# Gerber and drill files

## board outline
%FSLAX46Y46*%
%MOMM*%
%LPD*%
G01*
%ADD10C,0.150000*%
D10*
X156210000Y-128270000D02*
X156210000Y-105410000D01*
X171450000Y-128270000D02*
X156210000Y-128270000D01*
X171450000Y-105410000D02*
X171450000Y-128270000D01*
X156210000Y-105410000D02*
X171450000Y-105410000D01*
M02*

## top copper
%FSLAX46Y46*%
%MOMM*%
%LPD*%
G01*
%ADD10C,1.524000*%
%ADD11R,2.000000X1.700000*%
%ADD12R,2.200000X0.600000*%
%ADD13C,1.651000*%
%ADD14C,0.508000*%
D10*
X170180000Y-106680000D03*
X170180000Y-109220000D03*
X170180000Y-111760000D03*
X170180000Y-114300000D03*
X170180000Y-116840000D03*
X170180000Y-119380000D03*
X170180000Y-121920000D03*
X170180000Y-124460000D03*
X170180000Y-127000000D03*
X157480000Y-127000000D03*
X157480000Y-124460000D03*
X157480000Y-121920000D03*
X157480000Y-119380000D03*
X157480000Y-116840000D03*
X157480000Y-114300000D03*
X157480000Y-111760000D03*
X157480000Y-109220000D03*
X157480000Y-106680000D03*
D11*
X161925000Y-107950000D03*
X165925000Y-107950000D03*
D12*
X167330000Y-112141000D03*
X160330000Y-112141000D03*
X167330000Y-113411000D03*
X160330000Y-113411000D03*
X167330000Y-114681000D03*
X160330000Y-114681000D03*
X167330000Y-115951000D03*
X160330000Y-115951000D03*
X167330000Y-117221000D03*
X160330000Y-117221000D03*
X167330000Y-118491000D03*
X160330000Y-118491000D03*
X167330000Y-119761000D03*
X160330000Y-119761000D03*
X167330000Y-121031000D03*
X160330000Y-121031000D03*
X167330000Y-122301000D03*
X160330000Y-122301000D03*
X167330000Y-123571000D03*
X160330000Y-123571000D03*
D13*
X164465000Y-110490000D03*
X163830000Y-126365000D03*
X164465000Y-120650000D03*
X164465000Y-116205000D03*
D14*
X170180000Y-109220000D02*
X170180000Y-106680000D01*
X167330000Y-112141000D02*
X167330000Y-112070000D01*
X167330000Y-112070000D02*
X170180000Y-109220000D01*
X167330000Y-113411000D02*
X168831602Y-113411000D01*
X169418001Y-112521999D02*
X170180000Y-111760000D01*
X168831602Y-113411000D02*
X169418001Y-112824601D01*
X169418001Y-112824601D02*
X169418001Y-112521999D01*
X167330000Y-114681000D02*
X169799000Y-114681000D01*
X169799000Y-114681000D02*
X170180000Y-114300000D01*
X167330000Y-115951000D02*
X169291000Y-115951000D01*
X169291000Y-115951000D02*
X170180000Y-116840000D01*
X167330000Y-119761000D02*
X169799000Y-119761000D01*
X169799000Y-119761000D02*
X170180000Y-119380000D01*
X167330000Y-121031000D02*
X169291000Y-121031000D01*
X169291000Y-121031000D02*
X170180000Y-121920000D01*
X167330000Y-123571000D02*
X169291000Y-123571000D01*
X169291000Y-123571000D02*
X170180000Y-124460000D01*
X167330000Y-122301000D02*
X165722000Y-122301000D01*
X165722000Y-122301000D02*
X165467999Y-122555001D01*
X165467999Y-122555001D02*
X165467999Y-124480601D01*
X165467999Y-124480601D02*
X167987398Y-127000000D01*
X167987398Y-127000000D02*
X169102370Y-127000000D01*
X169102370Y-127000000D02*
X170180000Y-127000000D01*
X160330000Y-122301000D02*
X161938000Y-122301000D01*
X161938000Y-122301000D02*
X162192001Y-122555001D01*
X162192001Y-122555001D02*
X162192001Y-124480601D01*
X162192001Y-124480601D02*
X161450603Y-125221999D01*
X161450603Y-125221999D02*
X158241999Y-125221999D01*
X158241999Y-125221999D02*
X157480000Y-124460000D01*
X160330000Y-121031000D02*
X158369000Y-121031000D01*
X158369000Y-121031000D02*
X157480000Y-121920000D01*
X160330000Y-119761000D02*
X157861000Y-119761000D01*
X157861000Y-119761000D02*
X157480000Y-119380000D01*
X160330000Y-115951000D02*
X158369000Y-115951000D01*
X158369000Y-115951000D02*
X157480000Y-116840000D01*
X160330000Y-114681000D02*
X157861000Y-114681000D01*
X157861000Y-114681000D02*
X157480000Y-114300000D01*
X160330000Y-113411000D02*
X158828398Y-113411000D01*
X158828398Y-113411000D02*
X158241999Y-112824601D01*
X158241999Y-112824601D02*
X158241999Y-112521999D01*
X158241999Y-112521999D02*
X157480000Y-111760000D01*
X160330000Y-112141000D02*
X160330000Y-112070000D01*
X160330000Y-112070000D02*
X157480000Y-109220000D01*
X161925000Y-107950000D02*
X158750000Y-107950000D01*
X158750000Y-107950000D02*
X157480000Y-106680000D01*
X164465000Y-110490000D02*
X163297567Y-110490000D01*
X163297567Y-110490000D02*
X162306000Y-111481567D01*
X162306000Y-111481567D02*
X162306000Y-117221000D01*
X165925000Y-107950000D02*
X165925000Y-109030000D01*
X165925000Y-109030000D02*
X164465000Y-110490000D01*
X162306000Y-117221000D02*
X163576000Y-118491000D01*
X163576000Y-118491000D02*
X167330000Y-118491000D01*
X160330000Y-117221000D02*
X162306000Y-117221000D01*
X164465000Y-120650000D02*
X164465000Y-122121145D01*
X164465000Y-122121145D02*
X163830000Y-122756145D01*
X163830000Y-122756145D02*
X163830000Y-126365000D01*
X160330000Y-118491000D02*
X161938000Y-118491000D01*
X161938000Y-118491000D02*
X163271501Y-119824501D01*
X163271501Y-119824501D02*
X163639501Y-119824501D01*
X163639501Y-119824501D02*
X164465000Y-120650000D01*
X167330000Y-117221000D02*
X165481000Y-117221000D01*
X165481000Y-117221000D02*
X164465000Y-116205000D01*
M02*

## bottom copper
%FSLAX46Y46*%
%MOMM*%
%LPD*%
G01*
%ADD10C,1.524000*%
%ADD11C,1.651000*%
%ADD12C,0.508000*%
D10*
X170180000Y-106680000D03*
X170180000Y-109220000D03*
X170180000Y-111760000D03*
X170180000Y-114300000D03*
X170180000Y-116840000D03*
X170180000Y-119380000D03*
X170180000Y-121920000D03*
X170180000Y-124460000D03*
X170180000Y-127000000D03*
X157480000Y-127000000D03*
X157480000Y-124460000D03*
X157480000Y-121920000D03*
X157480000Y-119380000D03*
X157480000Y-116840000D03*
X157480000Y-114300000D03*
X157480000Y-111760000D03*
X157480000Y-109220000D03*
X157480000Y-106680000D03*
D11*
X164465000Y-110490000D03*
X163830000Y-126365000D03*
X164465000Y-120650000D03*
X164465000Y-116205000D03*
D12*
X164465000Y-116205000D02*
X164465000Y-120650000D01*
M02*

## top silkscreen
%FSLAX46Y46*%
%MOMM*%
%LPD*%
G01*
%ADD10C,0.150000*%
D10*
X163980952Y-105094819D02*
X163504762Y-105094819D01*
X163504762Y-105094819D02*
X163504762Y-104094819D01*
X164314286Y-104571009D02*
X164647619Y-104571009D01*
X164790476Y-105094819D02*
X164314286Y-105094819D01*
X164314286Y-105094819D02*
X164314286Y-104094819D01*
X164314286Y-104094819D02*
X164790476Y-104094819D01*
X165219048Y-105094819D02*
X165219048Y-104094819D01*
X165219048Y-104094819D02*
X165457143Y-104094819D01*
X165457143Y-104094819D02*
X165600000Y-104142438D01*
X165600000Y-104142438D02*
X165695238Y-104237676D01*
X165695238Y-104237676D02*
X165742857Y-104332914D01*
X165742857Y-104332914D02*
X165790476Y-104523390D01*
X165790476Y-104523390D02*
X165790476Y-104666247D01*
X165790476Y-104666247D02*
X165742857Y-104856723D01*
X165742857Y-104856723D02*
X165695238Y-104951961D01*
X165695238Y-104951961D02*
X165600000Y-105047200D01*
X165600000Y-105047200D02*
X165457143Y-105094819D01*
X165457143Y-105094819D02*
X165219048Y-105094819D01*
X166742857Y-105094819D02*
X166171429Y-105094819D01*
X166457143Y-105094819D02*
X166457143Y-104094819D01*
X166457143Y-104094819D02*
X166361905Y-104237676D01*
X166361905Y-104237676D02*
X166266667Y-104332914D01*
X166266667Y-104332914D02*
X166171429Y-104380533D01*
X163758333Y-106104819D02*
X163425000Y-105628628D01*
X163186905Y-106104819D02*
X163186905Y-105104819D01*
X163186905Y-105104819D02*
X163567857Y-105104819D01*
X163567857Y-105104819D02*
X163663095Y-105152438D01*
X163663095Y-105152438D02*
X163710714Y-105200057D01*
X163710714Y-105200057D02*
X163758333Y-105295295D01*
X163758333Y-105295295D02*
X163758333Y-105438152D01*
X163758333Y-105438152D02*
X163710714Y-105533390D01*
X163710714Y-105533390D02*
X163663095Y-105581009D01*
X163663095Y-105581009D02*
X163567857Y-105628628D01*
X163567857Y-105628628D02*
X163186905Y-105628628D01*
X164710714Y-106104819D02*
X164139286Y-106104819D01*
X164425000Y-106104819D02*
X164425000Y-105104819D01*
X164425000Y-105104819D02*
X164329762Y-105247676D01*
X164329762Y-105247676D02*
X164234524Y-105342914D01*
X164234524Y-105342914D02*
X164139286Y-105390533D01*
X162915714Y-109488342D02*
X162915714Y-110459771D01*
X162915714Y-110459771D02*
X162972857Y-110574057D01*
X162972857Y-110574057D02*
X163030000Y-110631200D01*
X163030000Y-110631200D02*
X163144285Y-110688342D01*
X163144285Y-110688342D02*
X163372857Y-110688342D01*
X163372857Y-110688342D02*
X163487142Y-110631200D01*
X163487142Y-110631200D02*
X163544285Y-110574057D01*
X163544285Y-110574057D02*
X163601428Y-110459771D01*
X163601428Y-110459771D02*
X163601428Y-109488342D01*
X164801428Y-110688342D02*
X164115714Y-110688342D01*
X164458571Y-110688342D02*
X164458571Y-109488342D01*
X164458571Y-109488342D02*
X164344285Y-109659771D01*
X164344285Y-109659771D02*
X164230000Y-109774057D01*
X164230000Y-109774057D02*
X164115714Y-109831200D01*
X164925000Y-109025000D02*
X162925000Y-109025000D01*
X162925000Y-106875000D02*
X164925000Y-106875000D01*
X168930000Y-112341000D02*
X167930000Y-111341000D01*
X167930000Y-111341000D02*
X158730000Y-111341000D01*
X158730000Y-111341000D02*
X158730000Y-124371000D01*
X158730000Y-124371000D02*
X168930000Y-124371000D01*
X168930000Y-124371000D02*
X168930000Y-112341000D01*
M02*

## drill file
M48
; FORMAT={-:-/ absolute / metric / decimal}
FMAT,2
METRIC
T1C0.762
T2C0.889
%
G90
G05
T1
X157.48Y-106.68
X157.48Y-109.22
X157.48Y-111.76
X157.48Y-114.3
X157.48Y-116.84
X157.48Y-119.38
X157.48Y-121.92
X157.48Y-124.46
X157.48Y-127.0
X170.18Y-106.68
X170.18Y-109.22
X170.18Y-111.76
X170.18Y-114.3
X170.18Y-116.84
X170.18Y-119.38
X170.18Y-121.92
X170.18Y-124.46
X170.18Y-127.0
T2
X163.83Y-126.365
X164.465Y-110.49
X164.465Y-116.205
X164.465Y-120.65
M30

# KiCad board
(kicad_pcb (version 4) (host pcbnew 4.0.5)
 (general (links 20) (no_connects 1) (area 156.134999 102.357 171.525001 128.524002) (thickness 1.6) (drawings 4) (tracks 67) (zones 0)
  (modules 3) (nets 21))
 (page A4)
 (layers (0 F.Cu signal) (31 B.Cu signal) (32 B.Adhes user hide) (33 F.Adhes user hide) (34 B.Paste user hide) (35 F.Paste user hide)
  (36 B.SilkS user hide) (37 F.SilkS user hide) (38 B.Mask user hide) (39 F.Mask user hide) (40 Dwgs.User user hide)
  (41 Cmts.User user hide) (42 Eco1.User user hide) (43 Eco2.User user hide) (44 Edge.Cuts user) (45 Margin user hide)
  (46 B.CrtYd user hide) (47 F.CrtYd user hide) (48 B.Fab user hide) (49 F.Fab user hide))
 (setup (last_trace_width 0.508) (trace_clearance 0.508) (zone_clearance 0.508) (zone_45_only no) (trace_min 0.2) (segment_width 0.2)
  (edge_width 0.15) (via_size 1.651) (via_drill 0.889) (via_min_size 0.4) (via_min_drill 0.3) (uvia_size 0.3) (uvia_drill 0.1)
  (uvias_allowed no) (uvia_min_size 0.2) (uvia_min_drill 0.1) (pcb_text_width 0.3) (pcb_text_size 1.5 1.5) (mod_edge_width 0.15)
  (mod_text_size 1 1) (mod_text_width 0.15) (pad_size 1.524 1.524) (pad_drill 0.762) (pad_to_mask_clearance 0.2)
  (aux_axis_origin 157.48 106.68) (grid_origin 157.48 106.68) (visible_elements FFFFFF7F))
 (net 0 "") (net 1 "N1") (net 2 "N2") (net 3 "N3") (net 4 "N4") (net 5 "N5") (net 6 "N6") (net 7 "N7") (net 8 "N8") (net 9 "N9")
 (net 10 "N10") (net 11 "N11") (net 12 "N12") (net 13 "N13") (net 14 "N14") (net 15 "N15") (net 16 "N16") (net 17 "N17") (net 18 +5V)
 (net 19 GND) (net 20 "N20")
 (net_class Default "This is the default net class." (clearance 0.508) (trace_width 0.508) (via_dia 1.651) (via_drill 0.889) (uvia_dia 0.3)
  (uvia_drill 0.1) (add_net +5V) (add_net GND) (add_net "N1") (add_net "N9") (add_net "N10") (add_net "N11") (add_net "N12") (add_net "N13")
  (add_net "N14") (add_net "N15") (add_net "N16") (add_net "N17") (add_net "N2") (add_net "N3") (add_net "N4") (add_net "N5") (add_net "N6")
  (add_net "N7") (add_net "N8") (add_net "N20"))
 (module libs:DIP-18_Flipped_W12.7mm (layer F.Cu) (at 165.1 104.14)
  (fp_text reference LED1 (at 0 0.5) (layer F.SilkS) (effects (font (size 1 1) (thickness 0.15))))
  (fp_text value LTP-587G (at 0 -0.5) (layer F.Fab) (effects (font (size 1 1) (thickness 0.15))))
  (pad 1 thru_hole circle (at 5.08 2.54) (size 1.524 1.524) (drill 0.762) (layers *.Cu *.Mask) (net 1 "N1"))
  (pad 2 thru_hole circle (at 5.08 5.08) (size 1.524 1.524) (drill 0.762) (layers *.Cu *.Mask) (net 1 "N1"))
  (pad 3 thru_hole circle (at 5.08 7.62) (size 1.524 1.524) (drill 0.762) (layers *.Cu *.Mask) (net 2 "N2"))
  (pad 4 thru_hole circle (at 5.08 10.16) (size 1.524 1.524) (drill 0.762) (layers *.Cu *.Mask) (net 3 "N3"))
  (pad 5 thru_hole circle (at 5.08 12.7) (size 1.524 1.524) (drill 0.762) (layers *.Cu *.Mask) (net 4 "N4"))
  (pad 6 thru_hole circle (at 5.08 15.24) (size 1.524 1.524) (drill 0.762) (layers *.Cu *.Mask) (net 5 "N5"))
  (pad 7 thru_hole circle (at 5.08 17.78) (size 1.524 1.524) (drill 0.762) (layers *.Cu *.Mask) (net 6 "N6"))
  (pad 8 thru_hole circle (at 5.08 20.32) (size 1.524 1.524) (drill 0.762) (layers *.Cu *.Mask) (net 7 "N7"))
  (pad 9 thru_hole circle (at 5.08 22.86) (size 1.524 1.524) (drill 0.762) (layers *.Cu *.Mask) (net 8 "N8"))
  (pad 10 thru_hole circle (at -7.62 22.86) (size 1.524 1.524) (drill 0.762) (layers *.Cu *.Mask) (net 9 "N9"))
  (pad 11 thru_hole circle (at -7.62 20.32) (size 1.524 1.524) (drill 0.762) (layers *.Cu *.Mask) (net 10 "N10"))
  (pad 12 thru_hole circle (at -7.62 17.78) (size 1.524 1.524) (drill 0.762) (layers *.Cu *.Mask) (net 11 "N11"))
  (pad 13 thru_hole circle (at -7.62 15.24) (size 1.524 1.524) (drill 0.762) (layers *.Cu *.Mask) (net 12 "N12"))
  (pad 14 thru_hole circle (at -7.62 12.7) (size 1.524 1.524) (drill 0.762) (layers *.Cu *.Mask) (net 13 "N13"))
  (pad 15 thru_hole circle (at -7.62 10.16) (size 1.524 1.524) (drill 0.762) (layers *.Cu *.Mask) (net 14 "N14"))
  (pad 16 thru_hole circle (at -7.62 7.62) (size 1.524 1.524) (drill 0.762) (layers *.Cu *.Mask) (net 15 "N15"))
  (pad 17 thru_hole circle (at -7.62 5.08) (size 1.524 1.524) (drill 0.762) (layers *.Cu *.Mask) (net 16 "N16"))
  (pad 18 thru_hole circle (at -7.62 2.54) (size 1.524 1.524) (drill 0.762) (layers *.Cu *.Mask) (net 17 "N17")))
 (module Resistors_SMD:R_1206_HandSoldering (layer F.Cu) (at 163.925 107.95)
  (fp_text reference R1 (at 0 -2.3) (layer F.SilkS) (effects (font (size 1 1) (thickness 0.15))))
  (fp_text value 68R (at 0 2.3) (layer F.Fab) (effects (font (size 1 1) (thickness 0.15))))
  (fp_line (start 1 1.075) (end -1 1.075) (layer F.SilkS) (width 0.15))
  (fp_line (start -1 -1.075) (end 1 -1.075) (layer F.SilkS) (width 0.15))
  (pad 1 smd rect (at -2 0) (size 2 1.7) (layers F.Cu F.Paste F.Mask) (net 17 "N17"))
  (pad 2 smd rect (at 2 0) (size 2 1.7) (layers F.Cu F.Paste F.Mask) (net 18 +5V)))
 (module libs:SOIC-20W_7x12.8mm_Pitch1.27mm (layer F.Cu) (at 163.83 117.856 270)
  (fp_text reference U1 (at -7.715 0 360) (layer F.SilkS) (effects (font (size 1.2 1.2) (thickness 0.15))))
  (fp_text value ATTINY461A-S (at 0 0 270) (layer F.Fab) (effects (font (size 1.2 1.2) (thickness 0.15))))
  (fp_line (start -5.515 -5.1) (end -6.515 -4.1) (layer F.SilkS) (width 0.15))
  (fp_line (start -6.515 -4.1) (end -6.515 5.1) (layer F.SilkS) (width 0.15))
  (fp_line (start -6.515 5.1) (end 6.515 5.1) (layer F.SilkS) (width 0.15))
  (fp_line (start 6.515 5.1) (end 6.515 -5.1) (layer F.SilkS) (width 0.15))
  (fp_line (start 6.515 -5.1) (end -5.515 -5.1) (layer F.SilkS) (width 0.15))
  (pad 20 smd rect (at -5.715 -3.5 270) (size 0.6 2.2) (layers F.Cu F.Paste F.Mask) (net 1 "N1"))
  (pad 1 smd rect (at -5.715 3.5 270) (size 0.6 2.2) (layers F.Cu F.Paste F.Mask) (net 16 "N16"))
  (pad 19 smd rect (at -4.445 -3.5 270) (size 0.6 2.2) (layers F.Cu F.Paste F.Mask) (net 2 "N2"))
  (pad 2 smd rect (at -4.445 3.5 270) (size 0.6 2.2) (layers F.Cu F.Paste F.Mask) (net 15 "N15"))
  (pad 18 smd rect (at -3.175 -3.5 270) (size 0.6 2.2) (layers F.Cu F.Paste F.Mask) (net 3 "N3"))
  (pad 3 smd rect (at -3.175 3.5 270) (size 0.6 2.2) (layers F.Cu F.Paste F.Mask) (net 14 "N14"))
  (pad 17 smd rect (at -1.905 -3.5 270) (size 0.6 2.2) (layers F.Cu F.Paste F.Mask) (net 4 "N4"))
  (pad 4 smd rect (at -1.905 3.5 270) (size 0.6 2.2) (layers F.Cu F.Paste F.Mask) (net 13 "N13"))
  (pad 16 smd rect (at -0.635 -3.5 270) (size 0.6 2.2) (layers F.Cu F.Paste F.Mask) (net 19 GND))
  (pad 5 smd rect (at -0.635 3.5 270) (size 0.6 2.2) (layers F.Cu F.Paste F.Mask) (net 18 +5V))
  (pad 15 smd rect (at 0.635 -3.5 270) (size 0.6 2.2) (layers F.Cu F.Paste F.Mask) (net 18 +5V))
  (pad 6 smd rect (at 0.635 3.5 270) (size 0.6 2.2) (layers F.Cu F.Paste F.Mask) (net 19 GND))
  (pad 14 smd rect (at 1.905 -3.5 270) (size 0.6 2.2) (layers F.Cu F.Paste F.Mask) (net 5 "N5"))
  (pad 7 smd rect (at 1.905 3.5 270) (size 0.6 2.2) (layers F.Cu F.Paste F.Mask) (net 12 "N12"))
  (pad 13 smd rect (at 3.175 -3.5 270) (size 0.6 2.2) (layers F.Cu F.Paste F.Mask) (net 6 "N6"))
  (pad 8 smd rect (at 3.175 3.5 270) (size 0.6 2.2) (layers F.Cu F.Paste F.Mask) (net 11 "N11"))
  (pad 12 smd rect (at 4.445 -3.5 270) (size 0.6 2.2) (layers F.Cu F.Paste F.Mask) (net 8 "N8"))
  (pad 9 smd rect (at 4.445 3.5 270) (size 0.6 2.2) (layers F.Cu F.Paste F.Mask) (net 10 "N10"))
  (pad 11 smd rect (at 5.715 -3.5 270) (size 0.6 2.2) (layers F.Cu F.Paste F.Mask) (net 7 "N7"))
  (pad 10 smd rect (at 5.715 3.5 270) (size 0.6 2.2) (layers F.Cu F.Paste F.Mask) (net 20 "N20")))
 (gr_line (start 156.21 128.27) (end 156.21 105.41) (layer Edge.Cuts) (width 0.15))
 (gr_line (start 171.45 128.27) (end 156.21 128.27) (layer Edge.Cuts) (width 0.15))
 (gr_line (start 171.45 105.41) (end 171.45 128.27) (layer Edge.Cuts) (width 0.15))
 (gr_line (start 156.21 105.41) (end 171.45 105.41) (layer Edge.Cuts) (width 0.15))
 (segment (start 170.18 109.22) (end 170.18 106.68) (width 0.508) (layer F.Cu) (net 1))
 (segment (start 167.33 112.141) (end 167.33 112.07) (width 0.508) (layer F.Cu) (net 1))
 (segment (start 167.33 112.07) (end 170.18 109.22) (width 0.508) (layer F.Cu) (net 1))
 (segment (start 167.33 113.411) (end 168.831602 113.411) (width 0.508) (layer F.Cu) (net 2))
 (segment (start 169.418001 112.521999) (end 170.18 111.76) (width 0.508) (layer F.Cu) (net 2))
 (segment (start 168.831602 113.411) (end 169.418001 112.824601) (width 0.508) (layer F.Cu) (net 2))
 (segment (start 169.418001 112.824601) (end 169.418001 112.521999) (width 0.508) (layer F.Cu) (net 2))
 (segment (start 167.33 114.681) (end 169.799 114.681) (width 0.508) (layer F.Cu) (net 3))
 (segment (start 169.799 114.681) (end 170.18 114.3) (width 0.508) (layer F.Cu) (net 3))
 (segment (start 167.33 115.951) (end 169.291 115.951) (width 0.508) (layer F.Cu) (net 4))
 (segment (start 169.291 115.951) (end 170.18 116.84) (width 0.508) (layer F.Cu) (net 4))
 (segment (start 167.33 119.761) (end 169.799 119.761) (width 0.508) (layer F.Cu) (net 5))
 (segment (start 169.799 119.761) (end 170.18 119.38) (width 0.508) (layer F.Cu) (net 5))
 (segment (start 167.33 121.031) (end 169.291 121.031) (width 0.508) (layer F.Cu) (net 6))
 (segment (start 169.291 121.031) (end 170.18 121.92) (width 0.508) (layer F.Cu) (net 6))
 (segment (start 167.33 123.571) (end 169.291 123.571) (width 0.508) (layer F.Cu) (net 7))
 (segment (start 169.291 123.571) (end 170.18 124.46) (width 0.508) (layer F.Cu) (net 7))
 (segment (start 167.33 122.301) (end 165.722 122.301) (width 0.508) (layer F.Cu) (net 8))
 (segment (start 165.722 122.301) (end 165.467999 122.555001) (width 0.508) (layer F.Cu) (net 8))
 (segment (start 165.467999 122.555001) (end 165.467999 124.480601) (width 0.508) (layer F.Cu) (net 8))
 (segment (start 165.467999 124.480601) (end 167.987398 127) (width 0.508) (layer F.Cu) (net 8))
 (segment (start 167.987398 127) (end 169.10237 127) (width 0.508) (layer F.Cu) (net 8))
 (segment (start 169.10237 127) (end 170.18 127) (width 0.508) (layer F.Cu) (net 8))
 (segment (start 160.33 122.301) (end 161.938 122.301) (width 0.508) (layer F.Cu) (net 10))
 (segment (start 161.938 122.301) (end 162.192001 122.555001) (width 0.508) (layer F.Cu) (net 10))
 (segment (start 162.192001 122.555001) (end 162.192001 124.480601) (width 0.508) (layer F.Cu) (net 10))
 (segment (start 162.192001 124.480601) (end 161.450603 125.221999) (width 0.508) (layer F.Cu) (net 10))
 (segment (start 161.450603 125.221999) (end 158.241999 125.221999) (width 0.508) (layer F.Cu) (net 10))
 (segment (start 158.241999 125.221999) (end 157.48 124.46) (width 0.508) (layer F.Cu) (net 10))
 (segment (start 160.33 121.031) (end 158.369 121.031) (width 0.508) (layer F.Cu) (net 11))
 (segment (start 158.369 121.031) (end 157.48 121.92) (width 0.508) (layer F.Cu) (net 11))
 (segment (start 160.33 119.761) (end 157.861 119.761) (width 0.508) (layer F.Cu) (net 12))
 (segment (start 157.861 119.761) (end 157.48 119.38) (width 0.508) (layer F.Cu) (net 12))
 (segment (start 160.33 115.951) (end 158.369 115.951) (width 0.508) (layer F.Cu) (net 13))
 (segment (start 158.369 115.951) (end 157.48 116.84) (width 0.508) (layer F.Cu) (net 13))
 (segment (start 160.33 114.681) (end 157.861 114.681) (width 0.508) (layer F.Cu) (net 14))
 (segment (start 157.861 114.681) (end 157.48 114.3) (width 0.508) (layer F.Cu) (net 14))
 (segment (start 160.33 113.411) (end 158.828398 113.411) (width 0.508) (layer F.Cu) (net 15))
 (segment (start 158.828398 113.411) (end 158.241999 112.824601) (width 0.508) (layer F.Cu) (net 15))
 (segment (start 158.241999 112.824601) (end 158.241999 112.521999) (width 0.508) (layer F.Cu) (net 15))
 (segment (start 158.241999 112.521999) (end 157.48 111.76) (width 0.508) (layer F.Cu) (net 15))
 (segment (start 160.33 112.141) (end 160.33 112.07) (width 0.508) (layer F.Cu) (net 16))
 (segment (start 160.33 112.07) (end 157.48 109.22) (width 0.508) (layer F.Cu) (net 16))
 (segment (start 161.925 107.95) (end 158.75 107.95) (width 0.508) (layer F.Cu) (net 17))
 (segment (start 158.75 107.95) (end 157.48 106.68) (width 0.508) (layer F.Cu) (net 17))
 (segment (start 164.465 110.49) (end 163.297567 110.49) (width 0.508) (layer F.Cu) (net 18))
 (segment (start 163.297567 110.49) (end 162.306 111.481567) (width 0.508) (layer F.Cu) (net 18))
 (segment (start 162.306 111.481567) (end 162.306 117.221) (width 0.508) (layer F.Cu) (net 18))
 (segment (start 165.925 107.95) (end 165.925 109.03) (width 0.508) (layer F.Cu) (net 18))
 (segment (start 165.925 109.03) (end 164.465 110.49) (width 0.508) (layer F.Cu) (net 18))
 (segment (start 162.306 117.221) (end 163.576 118.491) (width 0.508) (layer F.Cu) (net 18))
 (segment (start 163.576 118.491) (end 167.33 118.491) (width 0.508) (layer F.Cu) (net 18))
 (segment (start 160.33 117.221) (end 162.306 117.221) (width 0.508) (layer F.Cu) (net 18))
 (segment (start 164.465 120.65) (end 164.465 122.121145) (width 0.508) (layer F.Cu) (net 19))
 (segment (start 164.465 122.121145) (end 163.83 122.756145) (width 0.508) (layer F.Cu) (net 19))
 (segment (start 163.83 122.756145) (end 163.83 126.365) (width 0.508) (layer F.Cu) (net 19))
 (segment (start 160.33 118.491) (end 161.938 118.491) (width 0.508) (layer F.Cu) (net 19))
 (segment (start 161.938 118.491) (end 163.271501 119.824501) (width 0.508) (layer F.Cu) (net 19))
 (segment (start 163.271501 119.824501) (end 163.639501 119.824501) (width 0.508) (layer F.Cu) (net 19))
 (segment (start 163.639501 119.824501) (end 164.465 120.65) (width 0.508) (layer F.Cu) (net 19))
 (segment (start 164.465 116.205) (end 164.465 120.65) (width 0.508) (layer B.Cu) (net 19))
 (segment (start 167.33 117.221) (end 165.481 117.221) (width 0.508) (layer F.Cu) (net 19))
 (segment (start 165.481 117.221) (end 164.465 116.205) (width 0.508) (layer F.Cu) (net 19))
 (via (at 164.465 110.49) (size 1.651) (drill 0.889) (layers F.Cu B.Cu) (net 18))
 (via (at 163.83 126.365) (size 1.651) (drill 0.889) (layers F.Cu B.Cu) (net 19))
 (via (at 164.465 120.65) (size 1.651) (drill 0.889) (layers F.Cu B.Cu) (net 19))
 (via (at 164.465 116.205) (size 1.651) (drill 0.889) (layers F.Cu B.Cu) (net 19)))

